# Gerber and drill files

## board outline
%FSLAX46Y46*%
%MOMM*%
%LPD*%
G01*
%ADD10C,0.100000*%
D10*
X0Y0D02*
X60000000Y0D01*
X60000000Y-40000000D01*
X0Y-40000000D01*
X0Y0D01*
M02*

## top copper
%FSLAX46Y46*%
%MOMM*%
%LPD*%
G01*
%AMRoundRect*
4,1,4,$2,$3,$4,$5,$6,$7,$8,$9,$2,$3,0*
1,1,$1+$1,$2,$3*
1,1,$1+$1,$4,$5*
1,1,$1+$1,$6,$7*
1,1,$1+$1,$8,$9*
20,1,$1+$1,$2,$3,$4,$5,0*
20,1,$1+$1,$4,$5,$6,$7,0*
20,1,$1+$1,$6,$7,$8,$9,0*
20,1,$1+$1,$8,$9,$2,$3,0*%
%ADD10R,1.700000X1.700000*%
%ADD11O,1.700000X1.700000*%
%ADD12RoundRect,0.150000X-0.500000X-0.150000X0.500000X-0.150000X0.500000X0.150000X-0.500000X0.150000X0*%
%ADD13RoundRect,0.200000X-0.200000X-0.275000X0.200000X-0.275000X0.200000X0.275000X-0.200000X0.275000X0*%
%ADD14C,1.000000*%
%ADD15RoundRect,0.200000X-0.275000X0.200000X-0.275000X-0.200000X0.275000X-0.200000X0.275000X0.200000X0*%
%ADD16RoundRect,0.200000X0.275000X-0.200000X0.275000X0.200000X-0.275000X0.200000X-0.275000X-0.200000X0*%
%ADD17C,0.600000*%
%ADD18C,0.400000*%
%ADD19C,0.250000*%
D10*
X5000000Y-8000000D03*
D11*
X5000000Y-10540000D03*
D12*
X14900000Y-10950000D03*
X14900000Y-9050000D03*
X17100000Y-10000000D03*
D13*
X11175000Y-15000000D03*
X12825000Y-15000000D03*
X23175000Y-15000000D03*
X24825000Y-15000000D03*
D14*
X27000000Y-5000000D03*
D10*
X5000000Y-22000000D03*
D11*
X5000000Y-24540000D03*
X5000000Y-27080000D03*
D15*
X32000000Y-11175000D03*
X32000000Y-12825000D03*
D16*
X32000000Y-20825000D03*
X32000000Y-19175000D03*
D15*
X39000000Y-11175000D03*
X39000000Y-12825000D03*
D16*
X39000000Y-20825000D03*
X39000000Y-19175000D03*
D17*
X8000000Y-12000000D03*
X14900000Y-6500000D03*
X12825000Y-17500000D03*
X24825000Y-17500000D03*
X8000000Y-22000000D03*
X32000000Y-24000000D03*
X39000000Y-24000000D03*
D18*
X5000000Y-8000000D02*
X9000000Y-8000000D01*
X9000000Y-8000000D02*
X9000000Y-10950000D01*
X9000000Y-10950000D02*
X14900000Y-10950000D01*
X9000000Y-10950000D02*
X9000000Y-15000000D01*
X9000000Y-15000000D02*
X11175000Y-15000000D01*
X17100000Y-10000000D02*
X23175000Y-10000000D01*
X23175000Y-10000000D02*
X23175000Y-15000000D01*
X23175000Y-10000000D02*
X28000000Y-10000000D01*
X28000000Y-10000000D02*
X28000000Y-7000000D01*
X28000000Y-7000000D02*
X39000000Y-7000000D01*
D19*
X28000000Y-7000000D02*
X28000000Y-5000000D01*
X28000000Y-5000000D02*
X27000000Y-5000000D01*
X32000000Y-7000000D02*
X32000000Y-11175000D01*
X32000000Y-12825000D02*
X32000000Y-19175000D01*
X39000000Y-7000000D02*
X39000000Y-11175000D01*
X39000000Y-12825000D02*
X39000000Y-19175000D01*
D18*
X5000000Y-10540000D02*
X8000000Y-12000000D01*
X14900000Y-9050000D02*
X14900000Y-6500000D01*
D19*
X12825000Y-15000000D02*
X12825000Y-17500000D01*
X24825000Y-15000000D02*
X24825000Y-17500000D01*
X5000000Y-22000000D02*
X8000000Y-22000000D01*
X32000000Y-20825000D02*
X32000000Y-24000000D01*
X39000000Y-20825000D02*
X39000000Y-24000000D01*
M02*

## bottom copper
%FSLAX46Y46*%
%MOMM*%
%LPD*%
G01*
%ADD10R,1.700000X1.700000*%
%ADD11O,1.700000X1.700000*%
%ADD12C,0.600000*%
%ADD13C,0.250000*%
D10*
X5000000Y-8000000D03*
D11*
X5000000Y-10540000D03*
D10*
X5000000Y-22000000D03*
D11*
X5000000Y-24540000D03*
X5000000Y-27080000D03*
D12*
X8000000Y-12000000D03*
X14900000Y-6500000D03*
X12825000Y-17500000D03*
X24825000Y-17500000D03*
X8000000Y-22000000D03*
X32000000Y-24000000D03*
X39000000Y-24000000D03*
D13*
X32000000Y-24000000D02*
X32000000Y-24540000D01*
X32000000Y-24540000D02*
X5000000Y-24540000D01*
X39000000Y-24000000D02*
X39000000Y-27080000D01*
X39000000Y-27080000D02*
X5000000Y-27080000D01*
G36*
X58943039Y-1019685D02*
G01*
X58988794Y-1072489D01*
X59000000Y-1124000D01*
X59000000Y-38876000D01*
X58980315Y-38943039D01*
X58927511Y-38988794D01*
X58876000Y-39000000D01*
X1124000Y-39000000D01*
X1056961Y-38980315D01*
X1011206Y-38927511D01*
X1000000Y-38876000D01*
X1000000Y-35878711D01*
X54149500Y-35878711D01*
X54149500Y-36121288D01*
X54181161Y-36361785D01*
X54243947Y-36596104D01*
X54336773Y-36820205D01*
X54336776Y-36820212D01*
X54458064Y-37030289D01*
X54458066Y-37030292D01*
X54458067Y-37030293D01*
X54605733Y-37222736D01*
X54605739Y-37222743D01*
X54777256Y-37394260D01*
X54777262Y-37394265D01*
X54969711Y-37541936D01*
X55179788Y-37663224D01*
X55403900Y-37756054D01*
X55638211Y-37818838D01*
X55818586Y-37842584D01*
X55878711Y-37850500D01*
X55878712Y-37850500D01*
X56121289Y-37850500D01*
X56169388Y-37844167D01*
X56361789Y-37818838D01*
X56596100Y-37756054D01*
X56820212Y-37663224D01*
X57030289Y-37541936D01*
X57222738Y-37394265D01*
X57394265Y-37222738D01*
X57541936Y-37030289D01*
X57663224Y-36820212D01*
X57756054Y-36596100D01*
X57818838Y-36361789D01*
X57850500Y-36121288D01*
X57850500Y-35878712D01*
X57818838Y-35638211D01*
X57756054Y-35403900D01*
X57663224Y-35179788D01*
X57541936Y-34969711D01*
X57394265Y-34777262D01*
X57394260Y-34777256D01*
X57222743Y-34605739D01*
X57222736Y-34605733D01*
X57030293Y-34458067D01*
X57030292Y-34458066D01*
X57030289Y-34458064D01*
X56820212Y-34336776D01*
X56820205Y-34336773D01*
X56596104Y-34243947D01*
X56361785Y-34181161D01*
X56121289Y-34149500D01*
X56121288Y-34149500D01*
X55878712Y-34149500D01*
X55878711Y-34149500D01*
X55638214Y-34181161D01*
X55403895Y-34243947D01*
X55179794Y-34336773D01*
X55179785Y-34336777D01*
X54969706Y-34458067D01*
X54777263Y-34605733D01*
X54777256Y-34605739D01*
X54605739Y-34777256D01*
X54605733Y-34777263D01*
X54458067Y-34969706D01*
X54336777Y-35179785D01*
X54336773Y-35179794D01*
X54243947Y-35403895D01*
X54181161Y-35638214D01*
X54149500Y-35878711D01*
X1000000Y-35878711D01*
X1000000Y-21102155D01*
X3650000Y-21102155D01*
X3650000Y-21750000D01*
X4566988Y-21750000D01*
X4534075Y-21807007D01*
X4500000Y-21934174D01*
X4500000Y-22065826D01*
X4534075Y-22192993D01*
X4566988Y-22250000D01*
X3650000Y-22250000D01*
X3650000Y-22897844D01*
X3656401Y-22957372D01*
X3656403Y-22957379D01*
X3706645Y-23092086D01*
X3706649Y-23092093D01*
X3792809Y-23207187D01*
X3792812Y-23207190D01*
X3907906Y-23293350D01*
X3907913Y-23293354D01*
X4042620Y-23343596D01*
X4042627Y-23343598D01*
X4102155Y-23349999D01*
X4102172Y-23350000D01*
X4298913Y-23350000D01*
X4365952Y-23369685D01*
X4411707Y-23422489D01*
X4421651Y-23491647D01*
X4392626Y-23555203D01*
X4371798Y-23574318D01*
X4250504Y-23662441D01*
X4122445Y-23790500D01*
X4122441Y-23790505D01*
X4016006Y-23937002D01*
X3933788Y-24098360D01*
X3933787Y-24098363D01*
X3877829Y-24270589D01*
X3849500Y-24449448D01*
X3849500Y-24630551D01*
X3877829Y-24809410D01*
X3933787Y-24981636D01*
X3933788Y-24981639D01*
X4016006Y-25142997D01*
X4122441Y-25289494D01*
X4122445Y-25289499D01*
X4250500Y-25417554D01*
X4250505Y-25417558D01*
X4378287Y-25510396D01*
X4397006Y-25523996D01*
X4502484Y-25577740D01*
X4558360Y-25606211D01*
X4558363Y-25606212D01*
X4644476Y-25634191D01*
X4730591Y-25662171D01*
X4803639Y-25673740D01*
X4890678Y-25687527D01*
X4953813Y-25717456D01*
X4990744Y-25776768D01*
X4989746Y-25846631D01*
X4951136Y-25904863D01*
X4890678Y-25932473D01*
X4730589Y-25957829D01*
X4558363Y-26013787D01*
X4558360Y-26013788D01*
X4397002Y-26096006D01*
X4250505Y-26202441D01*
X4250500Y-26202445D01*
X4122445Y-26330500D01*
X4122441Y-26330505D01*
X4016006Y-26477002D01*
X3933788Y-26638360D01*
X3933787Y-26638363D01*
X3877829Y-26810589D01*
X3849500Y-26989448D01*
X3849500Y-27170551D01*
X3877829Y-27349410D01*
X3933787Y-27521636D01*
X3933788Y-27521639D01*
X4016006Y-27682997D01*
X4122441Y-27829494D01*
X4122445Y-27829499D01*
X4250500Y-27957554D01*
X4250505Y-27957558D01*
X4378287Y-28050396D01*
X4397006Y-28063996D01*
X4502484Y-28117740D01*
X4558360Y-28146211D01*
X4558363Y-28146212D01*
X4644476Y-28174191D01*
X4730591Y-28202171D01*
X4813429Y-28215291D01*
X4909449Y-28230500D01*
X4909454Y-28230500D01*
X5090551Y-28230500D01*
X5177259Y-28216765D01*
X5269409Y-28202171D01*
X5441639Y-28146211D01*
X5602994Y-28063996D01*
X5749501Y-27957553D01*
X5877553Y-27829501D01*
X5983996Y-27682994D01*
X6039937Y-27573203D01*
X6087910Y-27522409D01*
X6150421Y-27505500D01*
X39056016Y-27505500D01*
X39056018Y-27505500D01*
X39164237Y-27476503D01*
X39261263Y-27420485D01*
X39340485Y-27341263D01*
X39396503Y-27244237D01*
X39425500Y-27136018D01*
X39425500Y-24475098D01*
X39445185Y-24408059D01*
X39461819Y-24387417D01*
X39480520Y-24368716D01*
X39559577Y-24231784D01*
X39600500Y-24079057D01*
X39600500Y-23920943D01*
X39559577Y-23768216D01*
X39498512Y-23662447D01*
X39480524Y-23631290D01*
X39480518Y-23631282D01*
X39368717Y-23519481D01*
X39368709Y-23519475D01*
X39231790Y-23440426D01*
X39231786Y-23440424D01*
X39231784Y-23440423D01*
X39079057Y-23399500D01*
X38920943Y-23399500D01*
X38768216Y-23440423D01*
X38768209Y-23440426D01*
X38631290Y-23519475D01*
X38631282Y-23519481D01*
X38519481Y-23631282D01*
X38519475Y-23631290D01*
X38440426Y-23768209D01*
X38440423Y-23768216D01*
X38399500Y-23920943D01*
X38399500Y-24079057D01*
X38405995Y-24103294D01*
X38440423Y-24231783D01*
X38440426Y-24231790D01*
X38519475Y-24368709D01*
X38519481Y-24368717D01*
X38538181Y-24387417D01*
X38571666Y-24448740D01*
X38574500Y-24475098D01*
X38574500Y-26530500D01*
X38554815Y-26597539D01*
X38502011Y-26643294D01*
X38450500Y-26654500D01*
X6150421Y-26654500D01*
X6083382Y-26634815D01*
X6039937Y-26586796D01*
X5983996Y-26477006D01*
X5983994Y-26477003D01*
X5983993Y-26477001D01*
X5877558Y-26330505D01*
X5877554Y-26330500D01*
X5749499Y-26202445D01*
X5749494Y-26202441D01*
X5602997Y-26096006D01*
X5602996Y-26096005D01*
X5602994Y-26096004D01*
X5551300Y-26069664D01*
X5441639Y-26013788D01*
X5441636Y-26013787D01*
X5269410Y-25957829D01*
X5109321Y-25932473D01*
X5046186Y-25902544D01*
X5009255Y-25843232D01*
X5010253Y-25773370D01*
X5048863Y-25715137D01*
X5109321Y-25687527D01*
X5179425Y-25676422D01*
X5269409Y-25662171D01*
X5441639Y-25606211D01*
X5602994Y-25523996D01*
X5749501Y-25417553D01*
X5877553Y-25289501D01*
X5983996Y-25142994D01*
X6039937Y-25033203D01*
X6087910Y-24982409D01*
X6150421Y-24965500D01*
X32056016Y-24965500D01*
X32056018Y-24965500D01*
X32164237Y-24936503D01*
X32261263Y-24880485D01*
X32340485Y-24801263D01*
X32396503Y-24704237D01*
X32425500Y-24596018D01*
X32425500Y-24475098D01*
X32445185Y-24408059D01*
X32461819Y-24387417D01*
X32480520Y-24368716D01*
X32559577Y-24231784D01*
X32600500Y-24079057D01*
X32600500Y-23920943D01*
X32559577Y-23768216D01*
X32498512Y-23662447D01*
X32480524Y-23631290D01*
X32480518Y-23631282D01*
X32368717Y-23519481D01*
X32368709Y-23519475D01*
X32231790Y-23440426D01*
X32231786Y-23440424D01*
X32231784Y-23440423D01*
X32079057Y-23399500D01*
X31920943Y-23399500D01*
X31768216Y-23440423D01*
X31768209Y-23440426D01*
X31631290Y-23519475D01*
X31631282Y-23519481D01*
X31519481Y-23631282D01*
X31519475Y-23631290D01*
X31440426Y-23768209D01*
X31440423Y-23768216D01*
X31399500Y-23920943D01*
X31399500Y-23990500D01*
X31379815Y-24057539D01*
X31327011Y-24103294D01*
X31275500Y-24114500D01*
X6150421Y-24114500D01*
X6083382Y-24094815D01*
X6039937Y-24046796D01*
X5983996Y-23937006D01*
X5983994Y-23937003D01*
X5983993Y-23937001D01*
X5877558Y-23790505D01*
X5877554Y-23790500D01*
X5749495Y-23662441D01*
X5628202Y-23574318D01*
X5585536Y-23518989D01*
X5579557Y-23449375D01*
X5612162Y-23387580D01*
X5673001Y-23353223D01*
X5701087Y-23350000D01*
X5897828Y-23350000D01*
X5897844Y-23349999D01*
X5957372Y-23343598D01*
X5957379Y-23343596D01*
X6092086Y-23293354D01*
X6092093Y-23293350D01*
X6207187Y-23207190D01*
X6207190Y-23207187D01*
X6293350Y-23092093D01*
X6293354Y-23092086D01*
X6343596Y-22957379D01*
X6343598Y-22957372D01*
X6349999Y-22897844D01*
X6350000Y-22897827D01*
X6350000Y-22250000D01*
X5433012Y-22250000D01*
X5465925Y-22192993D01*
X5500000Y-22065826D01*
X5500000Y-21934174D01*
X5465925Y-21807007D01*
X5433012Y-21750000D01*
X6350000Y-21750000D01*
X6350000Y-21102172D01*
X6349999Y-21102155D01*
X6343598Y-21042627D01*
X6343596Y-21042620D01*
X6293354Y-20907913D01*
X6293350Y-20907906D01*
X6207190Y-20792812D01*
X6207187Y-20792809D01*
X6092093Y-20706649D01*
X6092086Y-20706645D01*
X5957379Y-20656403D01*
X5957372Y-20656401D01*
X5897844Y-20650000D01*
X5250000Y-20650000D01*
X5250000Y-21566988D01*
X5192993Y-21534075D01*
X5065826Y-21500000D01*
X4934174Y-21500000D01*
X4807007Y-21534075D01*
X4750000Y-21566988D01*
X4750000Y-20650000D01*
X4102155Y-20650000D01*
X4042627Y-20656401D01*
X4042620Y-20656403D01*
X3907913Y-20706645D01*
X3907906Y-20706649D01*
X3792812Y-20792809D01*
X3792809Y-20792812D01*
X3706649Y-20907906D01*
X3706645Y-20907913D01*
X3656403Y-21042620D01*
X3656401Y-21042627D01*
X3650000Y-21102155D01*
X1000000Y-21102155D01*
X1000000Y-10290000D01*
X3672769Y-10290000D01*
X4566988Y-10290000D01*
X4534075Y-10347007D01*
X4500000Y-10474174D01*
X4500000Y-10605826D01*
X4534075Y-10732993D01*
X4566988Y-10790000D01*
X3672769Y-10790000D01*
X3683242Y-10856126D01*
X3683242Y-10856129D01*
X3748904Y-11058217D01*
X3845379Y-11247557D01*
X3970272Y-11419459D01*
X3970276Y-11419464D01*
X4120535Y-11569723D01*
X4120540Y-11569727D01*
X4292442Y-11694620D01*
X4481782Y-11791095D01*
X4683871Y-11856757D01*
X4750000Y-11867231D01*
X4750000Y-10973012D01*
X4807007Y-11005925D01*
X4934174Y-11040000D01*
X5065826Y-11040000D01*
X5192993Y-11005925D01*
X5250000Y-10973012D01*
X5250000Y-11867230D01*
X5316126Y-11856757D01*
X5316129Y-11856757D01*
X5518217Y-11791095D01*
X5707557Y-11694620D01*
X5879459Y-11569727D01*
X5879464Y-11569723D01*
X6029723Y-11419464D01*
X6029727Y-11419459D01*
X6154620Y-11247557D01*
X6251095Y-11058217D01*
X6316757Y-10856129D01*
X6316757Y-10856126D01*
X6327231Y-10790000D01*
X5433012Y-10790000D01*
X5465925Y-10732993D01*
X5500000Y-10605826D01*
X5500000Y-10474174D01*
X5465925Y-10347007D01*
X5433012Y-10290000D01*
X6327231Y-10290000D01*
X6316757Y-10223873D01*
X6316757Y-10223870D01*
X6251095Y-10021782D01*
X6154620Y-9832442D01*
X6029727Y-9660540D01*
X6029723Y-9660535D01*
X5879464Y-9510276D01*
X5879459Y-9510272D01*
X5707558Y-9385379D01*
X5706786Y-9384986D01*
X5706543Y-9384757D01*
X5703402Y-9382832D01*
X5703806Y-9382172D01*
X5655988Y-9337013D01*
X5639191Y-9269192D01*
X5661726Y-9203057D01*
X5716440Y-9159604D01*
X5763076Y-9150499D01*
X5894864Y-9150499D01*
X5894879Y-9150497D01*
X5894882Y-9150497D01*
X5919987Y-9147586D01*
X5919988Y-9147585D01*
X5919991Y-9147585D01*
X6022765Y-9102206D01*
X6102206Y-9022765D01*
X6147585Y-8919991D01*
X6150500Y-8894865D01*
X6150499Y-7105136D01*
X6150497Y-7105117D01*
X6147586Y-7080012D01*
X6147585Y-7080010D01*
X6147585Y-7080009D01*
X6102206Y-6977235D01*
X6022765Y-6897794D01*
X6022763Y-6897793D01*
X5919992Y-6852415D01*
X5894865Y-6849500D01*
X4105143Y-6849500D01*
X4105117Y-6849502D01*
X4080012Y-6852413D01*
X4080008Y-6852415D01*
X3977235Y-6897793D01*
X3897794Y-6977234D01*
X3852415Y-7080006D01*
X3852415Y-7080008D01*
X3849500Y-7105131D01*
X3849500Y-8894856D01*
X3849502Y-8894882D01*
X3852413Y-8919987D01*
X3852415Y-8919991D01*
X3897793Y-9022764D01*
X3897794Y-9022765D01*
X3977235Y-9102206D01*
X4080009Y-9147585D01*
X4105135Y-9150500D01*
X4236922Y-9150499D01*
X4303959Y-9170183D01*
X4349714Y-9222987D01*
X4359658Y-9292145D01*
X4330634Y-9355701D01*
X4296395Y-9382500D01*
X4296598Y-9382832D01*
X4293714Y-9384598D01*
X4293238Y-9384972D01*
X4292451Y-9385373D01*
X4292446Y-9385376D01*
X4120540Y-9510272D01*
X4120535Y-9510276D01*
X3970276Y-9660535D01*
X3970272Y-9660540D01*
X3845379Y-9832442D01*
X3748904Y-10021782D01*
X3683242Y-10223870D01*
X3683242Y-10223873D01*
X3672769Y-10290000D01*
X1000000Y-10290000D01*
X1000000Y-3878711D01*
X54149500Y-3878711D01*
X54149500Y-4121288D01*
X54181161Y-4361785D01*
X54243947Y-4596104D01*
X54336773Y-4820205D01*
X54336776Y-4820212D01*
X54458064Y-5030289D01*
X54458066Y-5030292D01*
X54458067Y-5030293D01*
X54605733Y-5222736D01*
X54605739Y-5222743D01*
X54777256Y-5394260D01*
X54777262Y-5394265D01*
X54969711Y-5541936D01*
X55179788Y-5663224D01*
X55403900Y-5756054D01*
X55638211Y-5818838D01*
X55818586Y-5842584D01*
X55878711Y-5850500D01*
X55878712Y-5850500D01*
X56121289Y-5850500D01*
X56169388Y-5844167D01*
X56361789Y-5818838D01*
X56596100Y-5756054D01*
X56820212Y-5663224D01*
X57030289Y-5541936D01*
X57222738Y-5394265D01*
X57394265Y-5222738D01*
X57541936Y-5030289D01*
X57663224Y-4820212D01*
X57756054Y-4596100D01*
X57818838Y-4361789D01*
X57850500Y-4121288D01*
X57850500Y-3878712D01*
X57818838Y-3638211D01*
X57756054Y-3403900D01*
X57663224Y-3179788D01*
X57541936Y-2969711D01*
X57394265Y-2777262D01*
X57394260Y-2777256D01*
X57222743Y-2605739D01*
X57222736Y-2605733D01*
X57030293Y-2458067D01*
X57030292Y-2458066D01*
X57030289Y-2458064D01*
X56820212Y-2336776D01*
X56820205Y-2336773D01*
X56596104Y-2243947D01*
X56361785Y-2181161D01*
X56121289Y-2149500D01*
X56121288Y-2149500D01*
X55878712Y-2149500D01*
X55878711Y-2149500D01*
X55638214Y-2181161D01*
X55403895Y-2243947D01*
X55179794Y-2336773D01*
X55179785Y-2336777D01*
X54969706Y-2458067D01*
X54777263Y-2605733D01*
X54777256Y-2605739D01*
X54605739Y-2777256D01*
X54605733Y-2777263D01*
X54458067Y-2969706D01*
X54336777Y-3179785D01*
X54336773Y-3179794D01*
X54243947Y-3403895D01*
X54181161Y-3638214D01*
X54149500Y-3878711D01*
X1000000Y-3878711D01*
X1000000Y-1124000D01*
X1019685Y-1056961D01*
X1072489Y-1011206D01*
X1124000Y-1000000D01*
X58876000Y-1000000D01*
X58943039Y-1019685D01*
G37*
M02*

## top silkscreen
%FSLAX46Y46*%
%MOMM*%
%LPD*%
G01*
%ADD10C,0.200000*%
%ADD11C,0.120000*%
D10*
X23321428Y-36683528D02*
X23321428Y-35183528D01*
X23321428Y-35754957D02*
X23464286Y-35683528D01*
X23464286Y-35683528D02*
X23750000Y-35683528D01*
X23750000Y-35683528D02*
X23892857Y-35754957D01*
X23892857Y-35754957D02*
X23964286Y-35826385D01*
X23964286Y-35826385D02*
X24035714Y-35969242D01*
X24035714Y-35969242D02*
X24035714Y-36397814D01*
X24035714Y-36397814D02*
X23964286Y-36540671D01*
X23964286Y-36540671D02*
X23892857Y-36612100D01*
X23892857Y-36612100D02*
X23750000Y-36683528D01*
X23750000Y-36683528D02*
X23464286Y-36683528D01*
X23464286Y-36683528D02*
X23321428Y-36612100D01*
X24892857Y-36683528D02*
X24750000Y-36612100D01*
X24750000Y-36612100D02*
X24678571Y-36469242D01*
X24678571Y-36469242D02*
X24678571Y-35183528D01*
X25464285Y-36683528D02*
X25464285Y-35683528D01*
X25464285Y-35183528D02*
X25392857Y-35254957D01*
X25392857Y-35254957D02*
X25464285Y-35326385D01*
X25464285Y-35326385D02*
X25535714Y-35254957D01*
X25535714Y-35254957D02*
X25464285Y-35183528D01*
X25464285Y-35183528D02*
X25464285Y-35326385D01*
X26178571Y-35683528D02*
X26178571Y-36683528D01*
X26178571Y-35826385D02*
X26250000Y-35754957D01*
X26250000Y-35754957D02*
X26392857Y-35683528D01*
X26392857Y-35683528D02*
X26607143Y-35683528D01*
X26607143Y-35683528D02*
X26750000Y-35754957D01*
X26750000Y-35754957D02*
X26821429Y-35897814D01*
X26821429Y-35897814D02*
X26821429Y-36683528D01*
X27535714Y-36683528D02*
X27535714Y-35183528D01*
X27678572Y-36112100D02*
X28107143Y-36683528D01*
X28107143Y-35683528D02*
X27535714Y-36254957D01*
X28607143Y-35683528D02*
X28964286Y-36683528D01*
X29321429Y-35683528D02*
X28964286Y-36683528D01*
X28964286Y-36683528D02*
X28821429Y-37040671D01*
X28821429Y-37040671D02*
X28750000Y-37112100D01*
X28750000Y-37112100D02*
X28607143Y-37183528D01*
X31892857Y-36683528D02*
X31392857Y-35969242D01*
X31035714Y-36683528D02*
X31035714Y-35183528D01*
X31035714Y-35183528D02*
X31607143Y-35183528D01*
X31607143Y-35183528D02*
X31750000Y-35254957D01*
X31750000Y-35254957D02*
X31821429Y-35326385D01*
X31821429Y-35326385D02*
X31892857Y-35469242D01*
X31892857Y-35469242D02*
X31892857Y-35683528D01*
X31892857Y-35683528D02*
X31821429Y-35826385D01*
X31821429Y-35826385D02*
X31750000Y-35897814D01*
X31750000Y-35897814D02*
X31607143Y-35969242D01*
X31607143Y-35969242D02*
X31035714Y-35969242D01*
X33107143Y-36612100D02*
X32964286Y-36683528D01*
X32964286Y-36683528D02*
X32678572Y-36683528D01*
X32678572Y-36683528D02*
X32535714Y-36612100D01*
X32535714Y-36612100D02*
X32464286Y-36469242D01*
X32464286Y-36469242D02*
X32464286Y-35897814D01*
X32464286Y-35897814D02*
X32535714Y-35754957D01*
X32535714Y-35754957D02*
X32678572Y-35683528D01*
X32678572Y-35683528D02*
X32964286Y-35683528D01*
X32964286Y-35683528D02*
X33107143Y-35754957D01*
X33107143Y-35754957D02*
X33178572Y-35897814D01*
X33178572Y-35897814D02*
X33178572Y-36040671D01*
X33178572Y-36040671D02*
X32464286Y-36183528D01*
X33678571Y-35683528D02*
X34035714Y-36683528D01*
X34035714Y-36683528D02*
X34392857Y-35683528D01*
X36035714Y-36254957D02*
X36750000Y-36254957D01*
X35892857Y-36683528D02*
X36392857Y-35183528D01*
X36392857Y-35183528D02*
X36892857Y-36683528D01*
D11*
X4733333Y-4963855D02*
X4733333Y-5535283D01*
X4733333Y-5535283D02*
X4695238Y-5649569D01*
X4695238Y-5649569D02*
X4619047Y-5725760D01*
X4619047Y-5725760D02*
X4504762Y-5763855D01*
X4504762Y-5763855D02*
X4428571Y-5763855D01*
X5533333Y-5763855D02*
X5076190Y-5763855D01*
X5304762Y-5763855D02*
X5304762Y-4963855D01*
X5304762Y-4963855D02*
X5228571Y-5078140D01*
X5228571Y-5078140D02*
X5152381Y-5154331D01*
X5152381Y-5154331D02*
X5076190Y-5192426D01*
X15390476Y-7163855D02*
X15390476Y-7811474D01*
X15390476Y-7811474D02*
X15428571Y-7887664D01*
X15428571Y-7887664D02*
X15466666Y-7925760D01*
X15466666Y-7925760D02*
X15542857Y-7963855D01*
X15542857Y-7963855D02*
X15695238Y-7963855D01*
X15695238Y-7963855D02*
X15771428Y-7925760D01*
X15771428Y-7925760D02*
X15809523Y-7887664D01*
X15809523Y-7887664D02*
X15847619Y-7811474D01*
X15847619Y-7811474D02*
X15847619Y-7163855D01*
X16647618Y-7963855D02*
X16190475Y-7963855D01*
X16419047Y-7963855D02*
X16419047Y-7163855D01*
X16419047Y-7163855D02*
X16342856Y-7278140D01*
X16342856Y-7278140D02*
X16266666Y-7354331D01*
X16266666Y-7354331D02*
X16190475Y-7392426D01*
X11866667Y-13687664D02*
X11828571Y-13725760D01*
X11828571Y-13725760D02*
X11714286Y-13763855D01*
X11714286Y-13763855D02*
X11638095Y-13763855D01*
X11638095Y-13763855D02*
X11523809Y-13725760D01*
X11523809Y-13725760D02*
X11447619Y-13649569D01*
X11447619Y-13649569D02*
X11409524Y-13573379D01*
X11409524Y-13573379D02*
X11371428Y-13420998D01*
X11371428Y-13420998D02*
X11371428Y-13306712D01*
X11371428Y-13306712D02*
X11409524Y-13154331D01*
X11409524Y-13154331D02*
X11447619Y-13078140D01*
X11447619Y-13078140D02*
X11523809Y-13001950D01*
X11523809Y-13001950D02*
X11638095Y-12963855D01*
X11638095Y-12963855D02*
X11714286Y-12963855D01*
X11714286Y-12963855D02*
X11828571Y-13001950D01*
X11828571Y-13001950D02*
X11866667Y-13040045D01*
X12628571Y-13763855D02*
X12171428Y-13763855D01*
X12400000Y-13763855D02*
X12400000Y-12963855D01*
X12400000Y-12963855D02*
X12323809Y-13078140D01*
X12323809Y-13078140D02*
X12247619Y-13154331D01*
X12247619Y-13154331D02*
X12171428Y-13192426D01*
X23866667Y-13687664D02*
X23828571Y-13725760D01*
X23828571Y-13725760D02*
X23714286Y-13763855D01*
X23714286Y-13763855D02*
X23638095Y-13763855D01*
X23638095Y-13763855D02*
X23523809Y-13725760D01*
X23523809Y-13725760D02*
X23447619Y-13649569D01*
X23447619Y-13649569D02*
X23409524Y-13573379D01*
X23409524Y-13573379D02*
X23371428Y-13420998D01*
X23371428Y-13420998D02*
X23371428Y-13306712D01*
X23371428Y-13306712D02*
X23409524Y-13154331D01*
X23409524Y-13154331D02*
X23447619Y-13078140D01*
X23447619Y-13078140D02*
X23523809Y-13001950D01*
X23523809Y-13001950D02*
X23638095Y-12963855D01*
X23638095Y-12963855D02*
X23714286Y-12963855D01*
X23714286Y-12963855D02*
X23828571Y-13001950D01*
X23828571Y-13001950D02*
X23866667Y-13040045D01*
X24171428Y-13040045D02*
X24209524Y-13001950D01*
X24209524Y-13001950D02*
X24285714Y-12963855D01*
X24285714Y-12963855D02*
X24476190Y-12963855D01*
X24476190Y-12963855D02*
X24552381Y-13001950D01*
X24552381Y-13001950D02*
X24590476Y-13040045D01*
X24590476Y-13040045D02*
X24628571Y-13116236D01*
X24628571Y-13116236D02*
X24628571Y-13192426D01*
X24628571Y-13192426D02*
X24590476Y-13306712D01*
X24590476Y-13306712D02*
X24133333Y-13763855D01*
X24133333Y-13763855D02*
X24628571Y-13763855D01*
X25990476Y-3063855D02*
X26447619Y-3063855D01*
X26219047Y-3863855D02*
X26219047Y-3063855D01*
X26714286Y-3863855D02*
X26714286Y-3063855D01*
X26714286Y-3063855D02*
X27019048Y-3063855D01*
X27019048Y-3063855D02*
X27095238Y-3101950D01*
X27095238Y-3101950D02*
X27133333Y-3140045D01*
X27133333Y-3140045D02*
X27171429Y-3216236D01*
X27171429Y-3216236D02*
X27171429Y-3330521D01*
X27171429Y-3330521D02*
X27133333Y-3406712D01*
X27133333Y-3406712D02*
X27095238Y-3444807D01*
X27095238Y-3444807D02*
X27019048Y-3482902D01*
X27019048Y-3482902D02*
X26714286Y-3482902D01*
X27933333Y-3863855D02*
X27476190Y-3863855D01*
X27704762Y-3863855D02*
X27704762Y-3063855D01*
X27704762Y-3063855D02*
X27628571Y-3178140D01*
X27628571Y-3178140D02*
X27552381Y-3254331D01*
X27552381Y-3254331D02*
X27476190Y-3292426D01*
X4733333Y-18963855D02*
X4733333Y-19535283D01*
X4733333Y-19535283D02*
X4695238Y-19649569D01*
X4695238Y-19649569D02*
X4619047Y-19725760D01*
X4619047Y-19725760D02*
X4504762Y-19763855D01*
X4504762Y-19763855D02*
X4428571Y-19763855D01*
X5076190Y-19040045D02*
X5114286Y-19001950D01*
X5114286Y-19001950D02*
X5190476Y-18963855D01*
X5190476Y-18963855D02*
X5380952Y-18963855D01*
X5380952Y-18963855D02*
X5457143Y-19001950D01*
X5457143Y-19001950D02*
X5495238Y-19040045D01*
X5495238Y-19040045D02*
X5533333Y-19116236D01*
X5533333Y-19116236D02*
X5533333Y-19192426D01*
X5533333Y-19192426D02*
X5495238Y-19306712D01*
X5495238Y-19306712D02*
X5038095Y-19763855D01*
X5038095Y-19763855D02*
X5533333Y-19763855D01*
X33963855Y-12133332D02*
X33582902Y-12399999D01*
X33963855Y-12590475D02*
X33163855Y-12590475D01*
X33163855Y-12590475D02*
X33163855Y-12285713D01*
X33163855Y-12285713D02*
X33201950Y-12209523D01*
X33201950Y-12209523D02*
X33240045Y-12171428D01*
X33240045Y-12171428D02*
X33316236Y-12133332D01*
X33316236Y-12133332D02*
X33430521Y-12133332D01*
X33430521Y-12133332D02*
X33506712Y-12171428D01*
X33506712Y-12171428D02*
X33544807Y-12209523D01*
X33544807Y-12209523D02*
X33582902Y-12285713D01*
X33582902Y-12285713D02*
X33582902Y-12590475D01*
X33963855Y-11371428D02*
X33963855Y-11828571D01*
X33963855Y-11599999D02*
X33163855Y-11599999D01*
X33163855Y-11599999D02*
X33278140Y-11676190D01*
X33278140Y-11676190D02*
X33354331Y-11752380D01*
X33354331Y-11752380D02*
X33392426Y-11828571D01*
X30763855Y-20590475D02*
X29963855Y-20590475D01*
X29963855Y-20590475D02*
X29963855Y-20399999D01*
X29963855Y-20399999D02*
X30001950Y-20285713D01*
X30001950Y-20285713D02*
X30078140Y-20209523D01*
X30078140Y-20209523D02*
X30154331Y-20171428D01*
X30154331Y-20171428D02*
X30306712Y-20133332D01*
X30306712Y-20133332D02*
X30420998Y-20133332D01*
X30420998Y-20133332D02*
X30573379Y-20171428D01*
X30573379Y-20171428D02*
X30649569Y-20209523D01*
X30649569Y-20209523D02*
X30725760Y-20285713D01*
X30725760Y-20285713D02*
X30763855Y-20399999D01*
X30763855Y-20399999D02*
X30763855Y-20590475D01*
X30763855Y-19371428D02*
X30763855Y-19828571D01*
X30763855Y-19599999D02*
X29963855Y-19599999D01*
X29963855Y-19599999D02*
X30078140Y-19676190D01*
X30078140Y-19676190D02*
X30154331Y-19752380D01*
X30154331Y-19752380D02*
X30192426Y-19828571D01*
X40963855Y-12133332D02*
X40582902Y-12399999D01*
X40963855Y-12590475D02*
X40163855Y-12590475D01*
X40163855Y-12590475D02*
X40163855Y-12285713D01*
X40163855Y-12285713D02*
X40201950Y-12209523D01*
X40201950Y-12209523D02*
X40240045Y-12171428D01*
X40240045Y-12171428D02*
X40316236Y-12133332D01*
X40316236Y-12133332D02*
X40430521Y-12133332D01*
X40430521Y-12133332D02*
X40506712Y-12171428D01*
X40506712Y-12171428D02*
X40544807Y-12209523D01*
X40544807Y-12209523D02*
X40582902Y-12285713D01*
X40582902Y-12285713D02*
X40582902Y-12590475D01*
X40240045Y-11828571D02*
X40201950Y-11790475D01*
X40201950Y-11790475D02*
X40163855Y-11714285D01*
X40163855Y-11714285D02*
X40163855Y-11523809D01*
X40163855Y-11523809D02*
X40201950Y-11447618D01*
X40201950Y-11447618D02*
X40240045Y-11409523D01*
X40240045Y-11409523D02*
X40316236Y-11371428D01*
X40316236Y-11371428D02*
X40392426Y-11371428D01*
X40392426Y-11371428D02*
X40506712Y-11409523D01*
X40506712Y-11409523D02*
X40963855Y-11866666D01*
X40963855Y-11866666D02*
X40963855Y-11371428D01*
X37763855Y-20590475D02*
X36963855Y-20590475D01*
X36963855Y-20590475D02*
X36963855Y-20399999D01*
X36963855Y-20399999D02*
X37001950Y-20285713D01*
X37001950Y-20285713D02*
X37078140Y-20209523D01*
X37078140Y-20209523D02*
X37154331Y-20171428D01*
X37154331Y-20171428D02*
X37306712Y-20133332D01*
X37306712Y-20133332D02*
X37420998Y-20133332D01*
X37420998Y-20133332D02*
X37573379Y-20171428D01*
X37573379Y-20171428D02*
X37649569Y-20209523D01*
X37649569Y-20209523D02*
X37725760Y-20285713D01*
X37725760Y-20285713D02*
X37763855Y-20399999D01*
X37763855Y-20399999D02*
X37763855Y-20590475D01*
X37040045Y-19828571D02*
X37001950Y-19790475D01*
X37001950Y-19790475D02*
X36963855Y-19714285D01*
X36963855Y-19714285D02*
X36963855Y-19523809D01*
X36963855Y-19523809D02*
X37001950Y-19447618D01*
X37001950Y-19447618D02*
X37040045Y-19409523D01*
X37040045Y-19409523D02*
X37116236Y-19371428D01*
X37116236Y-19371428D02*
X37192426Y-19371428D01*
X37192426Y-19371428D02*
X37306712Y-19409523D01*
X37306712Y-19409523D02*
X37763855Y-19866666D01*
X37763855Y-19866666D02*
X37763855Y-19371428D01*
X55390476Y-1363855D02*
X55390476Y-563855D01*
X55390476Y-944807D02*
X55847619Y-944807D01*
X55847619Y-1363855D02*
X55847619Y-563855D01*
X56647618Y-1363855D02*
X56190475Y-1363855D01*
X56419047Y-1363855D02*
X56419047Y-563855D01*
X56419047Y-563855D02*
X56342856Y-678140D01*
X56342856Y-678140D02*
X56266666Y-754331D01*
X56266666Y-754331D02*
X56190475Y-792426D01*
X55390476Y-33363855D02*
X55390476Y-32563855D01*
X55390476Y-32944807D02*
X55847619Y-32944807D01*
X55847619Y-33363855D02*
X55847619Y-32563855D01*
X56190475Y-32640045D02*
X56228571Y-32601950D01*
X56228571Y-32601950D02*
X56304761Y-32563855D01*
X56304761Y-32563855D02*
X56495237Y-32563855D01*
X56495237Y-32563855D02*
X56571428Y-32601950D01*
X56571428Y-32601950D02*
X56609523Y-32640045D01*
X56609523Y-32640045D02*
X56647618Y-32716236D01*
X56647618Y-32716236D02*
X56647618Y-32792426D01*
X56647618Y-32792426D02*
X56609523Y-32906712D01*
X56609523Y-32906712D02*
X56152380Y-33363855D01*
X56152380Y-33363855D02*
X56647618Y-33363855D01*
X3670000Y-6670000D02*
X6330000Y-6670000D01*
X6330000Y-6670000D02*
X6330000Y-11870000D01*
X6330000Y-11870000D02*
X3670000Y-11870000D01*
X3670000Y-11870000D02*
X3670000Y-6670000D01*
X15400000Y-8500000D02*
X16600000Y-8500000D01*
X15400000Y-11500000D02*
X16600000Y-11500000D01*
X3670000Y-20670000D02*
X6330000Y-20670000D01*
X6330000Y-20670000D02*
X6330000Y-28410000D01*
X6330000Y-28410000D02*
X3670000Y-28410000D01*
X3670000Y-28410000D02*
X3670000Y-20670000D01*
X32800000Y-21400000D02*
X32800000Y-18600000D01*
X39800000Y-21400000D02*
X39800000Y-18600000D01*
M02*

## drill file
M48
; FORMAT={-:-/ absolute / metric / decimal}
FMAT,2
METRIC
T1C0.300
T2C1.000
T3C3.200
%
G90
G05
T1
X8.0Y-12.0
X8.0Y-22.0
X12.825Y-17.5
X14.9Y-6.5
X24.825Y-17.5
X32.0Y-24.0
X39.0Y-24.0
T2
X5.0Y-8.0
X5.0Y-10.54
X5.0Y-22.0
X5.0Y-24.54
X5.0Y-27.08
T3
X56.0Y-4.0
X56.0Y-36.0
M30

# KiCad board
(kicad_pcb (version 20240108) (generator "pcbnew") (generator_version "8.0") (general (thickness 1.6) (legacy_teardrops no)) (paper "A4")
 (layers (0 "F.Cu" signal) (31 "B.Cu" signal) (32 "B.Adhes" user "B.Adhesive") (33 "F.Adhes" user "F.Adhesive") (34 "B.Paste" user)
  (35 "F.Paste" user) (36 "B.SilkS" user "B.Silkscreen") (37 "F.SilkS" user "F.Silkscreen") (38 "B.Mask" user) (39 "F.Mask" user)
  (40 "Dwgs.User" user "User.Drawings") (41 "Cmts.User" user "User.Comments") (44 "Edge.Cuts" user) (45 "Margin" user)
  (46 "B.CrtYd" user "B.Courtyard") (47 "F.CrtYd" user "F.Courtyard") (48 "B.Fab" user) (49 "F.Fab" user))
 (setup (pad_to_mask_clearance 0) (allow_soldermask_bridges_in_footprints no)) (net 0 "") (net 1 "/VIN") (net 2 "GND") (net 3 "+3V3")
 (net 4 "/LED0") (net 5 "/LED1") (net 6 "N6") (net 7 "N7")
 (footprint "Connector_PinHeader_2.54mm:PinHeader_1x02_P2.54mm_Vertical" (layer "F.Cu") (at 5 8)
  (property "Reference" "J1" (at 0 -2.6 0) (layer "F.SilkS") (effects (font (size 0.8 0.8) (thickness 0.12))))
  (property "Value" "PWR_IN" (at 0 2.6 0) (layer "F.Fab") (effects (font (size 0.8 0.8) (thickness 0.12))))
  (fp_line (start -1.33 -1.33) (end 1.33 -1.33) (stroke (width 0.12) (type solid)) (layer "F.SilkS"))
  (fp_line (start 1.33 -1.33) (end 1.33 3.87) (stroke (width 0.12) (type solid)) (layer "F.SilkS"))
  (fp_line (start 1.33 3.87) (end -1.33 3.87) (stroke (width 0.12) (type solid)) (layer "F.SilkS"))
  (fp_line (start -1.33 3.87) (end -1.33 -1.33) (stroke (width 0.12) (type solid)) (layer "F.SilkS"))
  (pad "1" thru_hole rect (at 0 0) (size 1.7 1.7) (drill 1) (layers "*.Cu" "*.Mask") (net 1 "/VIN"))
  (pad "2" thru_hole oval (at 0 2.54) (size 1.7 1.7) (drill 1) (layers "*.Cu" "*.Mask") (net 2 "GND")))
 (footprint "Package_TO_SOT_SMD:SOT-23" (layer "F.Cu") (at 16 10)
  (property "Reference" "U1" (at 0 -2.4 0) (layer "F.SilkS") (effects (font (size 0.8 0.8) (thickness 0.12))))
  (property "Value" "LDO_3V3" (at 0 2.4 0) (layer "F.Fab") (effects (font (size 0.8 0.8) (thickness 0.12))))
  (fp_line (start -0.6 -1.5) (end 0.6 -1.5) (stroke (width 0.12) (type solid)) (layer "F.SilkS"))
  (fp_line (start -0.6 1.5) (end 0.6 1.5) (stroke (width 0.12) (type solid)) (layer "F.SilkS"))
  (pad "1" smd roundrect (at -1.1 0.95) (size 1.3 0.6) (layers "F.Cu" "F.Paste" "F.Mask") (roundrect_rratio 0.25) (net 1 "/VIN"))
  (pad "2" smd roundrect (at -1.1 -0.95) (size 1.3 0.6) (layers "F.Cu" "F.Paste" "F.Mask") (roundrect_rratio 0.25) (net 2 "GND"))
  (pad "3" smd roundrect (at 1.1 0) (size 1.3 0.6) (layers "F.Cu" "F.Paste" "F.Mask") (roundrect_rratio 0.25) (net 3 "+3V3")))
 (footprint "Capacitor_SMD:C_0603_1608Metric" (layer "F.Cu") (at 12 15)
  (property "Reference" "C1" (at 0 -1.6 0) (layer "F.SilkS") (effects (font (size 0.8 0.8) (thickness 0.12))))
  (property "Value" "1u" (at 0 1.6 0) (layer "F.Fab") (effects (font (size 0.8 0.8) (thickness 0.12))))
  (pad "1" smd roundrect (at -0.825 0) (size 0.8 0.95) (layers "F.Cu" "F.Paste" "F.Mask") (roundrect_rratio 0.25) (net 1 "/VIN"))
  (pad "2" smd roundrect (at 0.825 0) (size 0.8 0.95) (layers "F.Cu" "F.Paste" "F.Mask") (roundrect_rratio 0.25) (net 2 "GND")))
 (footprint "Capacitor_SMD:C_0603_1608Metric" (layer "F.Cu") (at 24 15)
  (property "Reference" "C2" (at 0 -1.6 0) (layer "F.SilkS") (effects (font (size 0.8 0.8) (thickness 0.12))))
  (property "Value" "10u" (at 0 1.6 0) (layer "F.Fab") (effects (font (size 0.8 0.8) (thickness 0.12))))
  (pad "1" smd roundrect (at -0.825 0) (size 0.8 0.95) (layers "F.Cu" "F.Paste" "F.Mask") (roundrect_rratio 0.25) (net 3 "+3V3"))
  (pad "2" smd roundrect (at 0.825 0) (size 0.8 0.95) (layers "F.Cu" "F.Paste" "F.Mask") (roundrect_rratio 0.25) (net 2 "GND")))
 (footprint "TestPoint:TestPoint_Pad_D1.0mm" (layer "F.Cu") (at 27 5)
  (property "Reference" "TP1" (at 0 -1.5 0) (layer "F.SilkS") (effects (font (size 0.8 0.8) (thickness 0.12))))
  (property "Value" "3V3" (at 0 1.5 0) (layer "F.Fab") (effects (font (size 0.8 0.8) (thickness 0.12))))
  (pad "1" smd circle (at 0 0) (size 1 1) (layers "F.Cu" "F.Mask") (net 3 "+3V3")))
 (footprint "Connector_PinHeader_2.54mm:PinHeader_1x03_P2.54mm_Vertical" (layer "F.Cu") (at 5 22)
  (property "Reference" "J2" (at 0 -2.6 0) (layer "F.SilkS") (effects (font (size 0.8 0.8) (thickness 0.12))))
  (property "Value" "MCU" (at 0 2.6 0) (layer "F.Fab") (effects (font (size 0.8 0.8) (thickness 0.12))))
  (fp_line (start -1.33 -1.33) (end 1.33 -1.33) (stroke (width 0.12) (type solid)) (layer "F.SilkS"))
  (fp_line (start 1.33 -1.33) (end 1.33 6.41) (stroke (width 0.12) (type solid)) (layer "F.SilkS"))
  (fp_line (start 1.33 6.41) (end -1.33 6.41) (stroke (width 0.12) (type solid)) (layer "F.SilkS"))
  (fp_line (start -1.33 6.41) (end -1.33 -1.33) (stroke (width 0.12) (type solid)) (layer "F.SilkS"))
  (pad "1" thru_hole rect (at 0 0) (size 1.7 1.7) (drill 1) (layers "*.Cu" "*.Mask") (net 2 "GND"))
  (pad "2" thru_hole oval (at 0 2.54) (size 1.7 1.7) (drill 1) (layers "*.Cu" "*.Mask") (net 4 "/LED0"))
  (pad "3" thru_hole oval (at 0 5.08) (size 1.7 1.7) (drill 1) (layers "*.Cu" "*.Mask") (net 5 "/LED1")))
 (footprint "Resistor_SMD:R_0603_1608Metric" (layer "F.Cu") (at 32 12 270)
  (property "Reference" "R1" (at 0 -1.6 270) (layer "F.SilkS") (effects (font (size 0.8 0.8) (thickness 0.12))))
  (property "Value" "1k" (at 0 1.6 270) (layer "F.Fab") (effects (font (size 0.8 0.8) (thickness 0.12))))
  (pad "1" smd roundrect (at -0.825 0 270) (size 0.8 0.95) (layers "F.Cu" "F.Paste" "F.Mask") (roundrect_rratio 0.25) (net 3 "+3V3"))
  (pad "2" smd roundrect (at 0.825 0 270) (size 0.8 0.95) (layers "F.Cu" "F.Paste" "F.Mask") (roundrect_rratio 0.25) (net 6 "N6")))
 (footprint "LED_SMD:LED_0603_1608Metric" (layer "F.Cu") (at 32 20 90)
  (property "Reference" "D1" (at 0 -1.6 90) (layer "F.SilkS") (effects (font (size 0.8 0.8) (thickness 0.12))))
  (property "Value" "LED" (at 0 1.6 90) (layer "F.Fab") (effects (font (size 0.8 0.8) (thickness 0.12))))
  (fp_line (start -1.4 0.8) (end 1.4 0.8) (stroke (width 0.12) (type solid)) (layer "F.SilkS"))
  (pad "1" smd roundrect (at -0.825 0 90) (size 0.8 0.95) (layers "F.Cu" "F.Paste" "F.Mask") (roundrect_rratio 0.25) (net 4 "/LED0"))
  (pad "2" smd roundrect (at 0.825 0 90) (size 0.8 0.95) (layers "F.Cu" "F.Paste" "F.Mask") (roundrect_rratio 0.25) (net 6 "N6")))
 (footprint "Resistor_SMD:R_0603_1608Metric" (layer "F.Cu") (at 39 12 270)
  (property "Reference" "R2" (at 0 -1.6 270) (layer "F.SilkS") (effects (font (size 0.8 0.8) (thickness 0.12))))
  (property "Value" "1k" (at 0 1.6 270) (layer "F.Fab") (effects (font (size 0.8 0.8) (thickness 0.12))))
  (pad "1" smd roundrect (at -0.825 0 270) (size 0.8 0.95) (layers "F.Cu" "F.Paste" "F.Mask") (roundrect_rratio 0.25) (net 3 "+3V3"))
  (pad "2" smd roundrect (at 0.825 0 270) (size 0.8 0.95) (layers "F.Cu" "F.Paste" "F.Mask") (roundrect_rratio 0.25) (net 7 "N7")))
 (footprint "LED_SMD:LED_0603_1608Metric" (layer "F.Cu") (at 39 20 90)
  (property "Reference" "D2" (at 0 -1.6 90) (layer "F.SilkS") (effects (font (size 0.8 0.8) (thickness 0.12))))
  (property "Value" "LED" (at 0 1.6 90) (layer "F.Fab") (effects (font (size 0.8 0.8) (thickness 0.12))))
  (fp_line (start -1.4 0.8) (end 1.4 0.8) (stroke (width 0.12) (type solid)) (layer "F.SilkS"))
  (pad "1" smd roundrect (at -0.825 0 90) (size 0.8 0.95) (layers "F.Cu" "F.Paste" "F.Mask") (roundrect_rratio 0.25) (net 5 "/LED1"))
  (pad "2" smd roundrect (at 0.825 0 90) (size 0.8 0.95) (layers "F.Cu" "F.Paste" "F.Mask") (roundrect_rratio 0.25) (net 7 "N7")))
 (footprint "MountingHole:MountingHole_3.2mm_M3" (layer "F.Cu") (at 56 4)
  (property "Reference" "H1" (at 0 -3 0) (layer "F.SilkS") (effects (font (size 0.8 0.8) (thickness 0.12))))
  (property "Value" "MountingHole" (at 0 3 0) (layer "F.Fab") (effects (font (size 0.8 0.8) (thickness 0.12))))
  (pad "" np_thru_hole circle (at 0 0) (size 3.2 3.2) (drill 3.2) (layers "*.Cu" "*.Mask")))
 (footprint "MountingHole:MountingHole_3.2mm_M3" (layer "F.Cu") (at 56 36)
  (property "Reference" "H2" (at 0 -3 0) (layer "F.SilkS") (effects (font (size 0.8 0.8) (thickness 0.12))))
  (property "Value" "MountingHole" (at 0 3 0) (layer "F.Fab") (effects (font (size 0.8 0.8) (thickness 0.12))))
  (pad "" np_thru_hole circle (at 0 0) (size 3.2 3.2) (drill 3.2) (layers "*.Cu" "*.Mask")))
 (segment (start 5 8) (end 9 8) (width 0.4) (layer "F.Cu") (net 1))
 (segment (start 9 8) (end 9 10.95) (width 0.4) (layer "F.Cu") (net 1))
 (segment (start 9 10.95) (end 14.9 10.95) (width 0.4) (layer "F.Cu") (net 1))
 (segment (start 9 10.95) (end 9 15) (width 0.4) (layer "F.Cu") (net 1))
 (segment (start 9 15) (end 11.175 15) (width 0.4) (layer "F.Cu") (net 1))
 (segment (start 17.1 10) (end 23.175 10) (width 0.4) (layer "F.Cu") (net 3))
 (segment (start 23.175 10) (end 23.175 15) (width 0.4) (layer "F.Cu") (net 3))
 (segment (start 23.175 10) (end 28 10) (width 0.4) (layer "F.Cu") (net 3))
 (segment (start 28 10) (end 28 7) (width 0.4) (layer "F.Cu") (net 3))
 (segment (start 28 7) (end 39 7) (width 0.4) (layer "F.Cu") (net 3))
 (segment (start 28 7) (end 28 5) (width 0.25) (layer "F.Cu") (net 3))
 (segment (start 28 5) (end 27 5) (width 0.25) (layer "F.Cu") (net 3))
 (segment (start 32 7) (end 32 11.175) (width 0.25) (layer "F.Cu") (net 3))
 (segment (start 32 12.825) (end 32 19.175) (width 0.25) (layer "F.Cu") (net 6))
 (segment (start 39 7) (end 39 11.175) (width 0.25) (layer "F.Cu") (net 3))
 (segment (start 39 12.825) (end 39 19.175) (width 0.25) (layer "F.Cu") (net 7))
 (segment (start 5 10.54) (end 8 12) (width 0.4) (layer "F.Cu") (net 2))
 (via (at 8 12) (size 0.6) (drill 0.3) (layers "F.Cu" "B.Cu") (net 2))
 (segment (start 14.9 9.05) (end 14.9 6.5) (width 0.4) (layer "F.Cu") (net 2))
 (via (at 14.9 6.5) (size 0.6) (drill 0.3) (layers "F.Cu" "B.Cu") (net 2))
 (segment (start 12.825 15) (end 12.825 17.5) (width 0.25) (layer "F.Cu") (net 2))
 (via (at 12.825 17.5) (size 0.6) (drill 0.3) (layers "F.Cu" "B.Cu") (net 2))
 (segment (start 24.825 15) (end 24.825 17.5) (width 0.25) (layer "F.Cu") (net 2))
 (via (at 24.825 17.5) (size 0.6) (drill 0.3) (layers "F.Cu" "B.Cu") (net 2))
 (segment (start 5 22) (end 8 22) (width 0.25) (layer "F.Cu") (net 2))
 (via (at 8 22) (size 0.6) (drill 0.3) (layers "F.Cu" "B.Cu") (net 2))
 (segment (start 32 20.825) (end 32 24) (width 0.25) (layer "F.Cu") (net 4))
 (via (at 32 24) (size 0.6) (drill 0.3) (layers "F.Cu" "B.Cu") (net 4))
 (segment (start 32 24) (end 32 24.54) (width 0.25) (layer "B.Cu") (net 4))
 (segment (start 32 24.54) (end 5 24.54) (width 0.25) (layer "B.Cu") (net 4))
 (segment (start 39 20.825) (end 39 24) (width 0.25) (layer "F.Cu") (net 5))
 (via (at 39 24) (size 0.6) (drill 0.3) (layers "F.Cu" "B.Cu") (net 5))
 (segment (start 39 24) (end 39 27.08) (width 0.25) (layer "B.Cu") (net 5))
 (segment (start 39 27.08) (end 5 27.08) (width 0.25) (layer "B.Cu") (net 5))
 (gr_rect (start 0 0) (end 60 40) (stroke (width 0.1) (type default)) (fill none) (layer "Edge.Cuts"))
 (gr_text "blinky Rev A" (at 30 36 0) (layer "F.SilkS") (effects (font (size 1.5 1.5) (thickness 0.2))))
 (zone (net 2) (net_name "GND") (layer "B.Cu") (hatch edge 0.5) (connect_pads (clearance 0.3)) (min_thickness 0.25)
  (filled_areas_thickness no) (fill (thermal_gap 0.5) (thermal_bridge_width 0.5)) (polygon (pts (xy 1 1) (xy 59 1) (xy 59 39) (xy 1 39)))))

